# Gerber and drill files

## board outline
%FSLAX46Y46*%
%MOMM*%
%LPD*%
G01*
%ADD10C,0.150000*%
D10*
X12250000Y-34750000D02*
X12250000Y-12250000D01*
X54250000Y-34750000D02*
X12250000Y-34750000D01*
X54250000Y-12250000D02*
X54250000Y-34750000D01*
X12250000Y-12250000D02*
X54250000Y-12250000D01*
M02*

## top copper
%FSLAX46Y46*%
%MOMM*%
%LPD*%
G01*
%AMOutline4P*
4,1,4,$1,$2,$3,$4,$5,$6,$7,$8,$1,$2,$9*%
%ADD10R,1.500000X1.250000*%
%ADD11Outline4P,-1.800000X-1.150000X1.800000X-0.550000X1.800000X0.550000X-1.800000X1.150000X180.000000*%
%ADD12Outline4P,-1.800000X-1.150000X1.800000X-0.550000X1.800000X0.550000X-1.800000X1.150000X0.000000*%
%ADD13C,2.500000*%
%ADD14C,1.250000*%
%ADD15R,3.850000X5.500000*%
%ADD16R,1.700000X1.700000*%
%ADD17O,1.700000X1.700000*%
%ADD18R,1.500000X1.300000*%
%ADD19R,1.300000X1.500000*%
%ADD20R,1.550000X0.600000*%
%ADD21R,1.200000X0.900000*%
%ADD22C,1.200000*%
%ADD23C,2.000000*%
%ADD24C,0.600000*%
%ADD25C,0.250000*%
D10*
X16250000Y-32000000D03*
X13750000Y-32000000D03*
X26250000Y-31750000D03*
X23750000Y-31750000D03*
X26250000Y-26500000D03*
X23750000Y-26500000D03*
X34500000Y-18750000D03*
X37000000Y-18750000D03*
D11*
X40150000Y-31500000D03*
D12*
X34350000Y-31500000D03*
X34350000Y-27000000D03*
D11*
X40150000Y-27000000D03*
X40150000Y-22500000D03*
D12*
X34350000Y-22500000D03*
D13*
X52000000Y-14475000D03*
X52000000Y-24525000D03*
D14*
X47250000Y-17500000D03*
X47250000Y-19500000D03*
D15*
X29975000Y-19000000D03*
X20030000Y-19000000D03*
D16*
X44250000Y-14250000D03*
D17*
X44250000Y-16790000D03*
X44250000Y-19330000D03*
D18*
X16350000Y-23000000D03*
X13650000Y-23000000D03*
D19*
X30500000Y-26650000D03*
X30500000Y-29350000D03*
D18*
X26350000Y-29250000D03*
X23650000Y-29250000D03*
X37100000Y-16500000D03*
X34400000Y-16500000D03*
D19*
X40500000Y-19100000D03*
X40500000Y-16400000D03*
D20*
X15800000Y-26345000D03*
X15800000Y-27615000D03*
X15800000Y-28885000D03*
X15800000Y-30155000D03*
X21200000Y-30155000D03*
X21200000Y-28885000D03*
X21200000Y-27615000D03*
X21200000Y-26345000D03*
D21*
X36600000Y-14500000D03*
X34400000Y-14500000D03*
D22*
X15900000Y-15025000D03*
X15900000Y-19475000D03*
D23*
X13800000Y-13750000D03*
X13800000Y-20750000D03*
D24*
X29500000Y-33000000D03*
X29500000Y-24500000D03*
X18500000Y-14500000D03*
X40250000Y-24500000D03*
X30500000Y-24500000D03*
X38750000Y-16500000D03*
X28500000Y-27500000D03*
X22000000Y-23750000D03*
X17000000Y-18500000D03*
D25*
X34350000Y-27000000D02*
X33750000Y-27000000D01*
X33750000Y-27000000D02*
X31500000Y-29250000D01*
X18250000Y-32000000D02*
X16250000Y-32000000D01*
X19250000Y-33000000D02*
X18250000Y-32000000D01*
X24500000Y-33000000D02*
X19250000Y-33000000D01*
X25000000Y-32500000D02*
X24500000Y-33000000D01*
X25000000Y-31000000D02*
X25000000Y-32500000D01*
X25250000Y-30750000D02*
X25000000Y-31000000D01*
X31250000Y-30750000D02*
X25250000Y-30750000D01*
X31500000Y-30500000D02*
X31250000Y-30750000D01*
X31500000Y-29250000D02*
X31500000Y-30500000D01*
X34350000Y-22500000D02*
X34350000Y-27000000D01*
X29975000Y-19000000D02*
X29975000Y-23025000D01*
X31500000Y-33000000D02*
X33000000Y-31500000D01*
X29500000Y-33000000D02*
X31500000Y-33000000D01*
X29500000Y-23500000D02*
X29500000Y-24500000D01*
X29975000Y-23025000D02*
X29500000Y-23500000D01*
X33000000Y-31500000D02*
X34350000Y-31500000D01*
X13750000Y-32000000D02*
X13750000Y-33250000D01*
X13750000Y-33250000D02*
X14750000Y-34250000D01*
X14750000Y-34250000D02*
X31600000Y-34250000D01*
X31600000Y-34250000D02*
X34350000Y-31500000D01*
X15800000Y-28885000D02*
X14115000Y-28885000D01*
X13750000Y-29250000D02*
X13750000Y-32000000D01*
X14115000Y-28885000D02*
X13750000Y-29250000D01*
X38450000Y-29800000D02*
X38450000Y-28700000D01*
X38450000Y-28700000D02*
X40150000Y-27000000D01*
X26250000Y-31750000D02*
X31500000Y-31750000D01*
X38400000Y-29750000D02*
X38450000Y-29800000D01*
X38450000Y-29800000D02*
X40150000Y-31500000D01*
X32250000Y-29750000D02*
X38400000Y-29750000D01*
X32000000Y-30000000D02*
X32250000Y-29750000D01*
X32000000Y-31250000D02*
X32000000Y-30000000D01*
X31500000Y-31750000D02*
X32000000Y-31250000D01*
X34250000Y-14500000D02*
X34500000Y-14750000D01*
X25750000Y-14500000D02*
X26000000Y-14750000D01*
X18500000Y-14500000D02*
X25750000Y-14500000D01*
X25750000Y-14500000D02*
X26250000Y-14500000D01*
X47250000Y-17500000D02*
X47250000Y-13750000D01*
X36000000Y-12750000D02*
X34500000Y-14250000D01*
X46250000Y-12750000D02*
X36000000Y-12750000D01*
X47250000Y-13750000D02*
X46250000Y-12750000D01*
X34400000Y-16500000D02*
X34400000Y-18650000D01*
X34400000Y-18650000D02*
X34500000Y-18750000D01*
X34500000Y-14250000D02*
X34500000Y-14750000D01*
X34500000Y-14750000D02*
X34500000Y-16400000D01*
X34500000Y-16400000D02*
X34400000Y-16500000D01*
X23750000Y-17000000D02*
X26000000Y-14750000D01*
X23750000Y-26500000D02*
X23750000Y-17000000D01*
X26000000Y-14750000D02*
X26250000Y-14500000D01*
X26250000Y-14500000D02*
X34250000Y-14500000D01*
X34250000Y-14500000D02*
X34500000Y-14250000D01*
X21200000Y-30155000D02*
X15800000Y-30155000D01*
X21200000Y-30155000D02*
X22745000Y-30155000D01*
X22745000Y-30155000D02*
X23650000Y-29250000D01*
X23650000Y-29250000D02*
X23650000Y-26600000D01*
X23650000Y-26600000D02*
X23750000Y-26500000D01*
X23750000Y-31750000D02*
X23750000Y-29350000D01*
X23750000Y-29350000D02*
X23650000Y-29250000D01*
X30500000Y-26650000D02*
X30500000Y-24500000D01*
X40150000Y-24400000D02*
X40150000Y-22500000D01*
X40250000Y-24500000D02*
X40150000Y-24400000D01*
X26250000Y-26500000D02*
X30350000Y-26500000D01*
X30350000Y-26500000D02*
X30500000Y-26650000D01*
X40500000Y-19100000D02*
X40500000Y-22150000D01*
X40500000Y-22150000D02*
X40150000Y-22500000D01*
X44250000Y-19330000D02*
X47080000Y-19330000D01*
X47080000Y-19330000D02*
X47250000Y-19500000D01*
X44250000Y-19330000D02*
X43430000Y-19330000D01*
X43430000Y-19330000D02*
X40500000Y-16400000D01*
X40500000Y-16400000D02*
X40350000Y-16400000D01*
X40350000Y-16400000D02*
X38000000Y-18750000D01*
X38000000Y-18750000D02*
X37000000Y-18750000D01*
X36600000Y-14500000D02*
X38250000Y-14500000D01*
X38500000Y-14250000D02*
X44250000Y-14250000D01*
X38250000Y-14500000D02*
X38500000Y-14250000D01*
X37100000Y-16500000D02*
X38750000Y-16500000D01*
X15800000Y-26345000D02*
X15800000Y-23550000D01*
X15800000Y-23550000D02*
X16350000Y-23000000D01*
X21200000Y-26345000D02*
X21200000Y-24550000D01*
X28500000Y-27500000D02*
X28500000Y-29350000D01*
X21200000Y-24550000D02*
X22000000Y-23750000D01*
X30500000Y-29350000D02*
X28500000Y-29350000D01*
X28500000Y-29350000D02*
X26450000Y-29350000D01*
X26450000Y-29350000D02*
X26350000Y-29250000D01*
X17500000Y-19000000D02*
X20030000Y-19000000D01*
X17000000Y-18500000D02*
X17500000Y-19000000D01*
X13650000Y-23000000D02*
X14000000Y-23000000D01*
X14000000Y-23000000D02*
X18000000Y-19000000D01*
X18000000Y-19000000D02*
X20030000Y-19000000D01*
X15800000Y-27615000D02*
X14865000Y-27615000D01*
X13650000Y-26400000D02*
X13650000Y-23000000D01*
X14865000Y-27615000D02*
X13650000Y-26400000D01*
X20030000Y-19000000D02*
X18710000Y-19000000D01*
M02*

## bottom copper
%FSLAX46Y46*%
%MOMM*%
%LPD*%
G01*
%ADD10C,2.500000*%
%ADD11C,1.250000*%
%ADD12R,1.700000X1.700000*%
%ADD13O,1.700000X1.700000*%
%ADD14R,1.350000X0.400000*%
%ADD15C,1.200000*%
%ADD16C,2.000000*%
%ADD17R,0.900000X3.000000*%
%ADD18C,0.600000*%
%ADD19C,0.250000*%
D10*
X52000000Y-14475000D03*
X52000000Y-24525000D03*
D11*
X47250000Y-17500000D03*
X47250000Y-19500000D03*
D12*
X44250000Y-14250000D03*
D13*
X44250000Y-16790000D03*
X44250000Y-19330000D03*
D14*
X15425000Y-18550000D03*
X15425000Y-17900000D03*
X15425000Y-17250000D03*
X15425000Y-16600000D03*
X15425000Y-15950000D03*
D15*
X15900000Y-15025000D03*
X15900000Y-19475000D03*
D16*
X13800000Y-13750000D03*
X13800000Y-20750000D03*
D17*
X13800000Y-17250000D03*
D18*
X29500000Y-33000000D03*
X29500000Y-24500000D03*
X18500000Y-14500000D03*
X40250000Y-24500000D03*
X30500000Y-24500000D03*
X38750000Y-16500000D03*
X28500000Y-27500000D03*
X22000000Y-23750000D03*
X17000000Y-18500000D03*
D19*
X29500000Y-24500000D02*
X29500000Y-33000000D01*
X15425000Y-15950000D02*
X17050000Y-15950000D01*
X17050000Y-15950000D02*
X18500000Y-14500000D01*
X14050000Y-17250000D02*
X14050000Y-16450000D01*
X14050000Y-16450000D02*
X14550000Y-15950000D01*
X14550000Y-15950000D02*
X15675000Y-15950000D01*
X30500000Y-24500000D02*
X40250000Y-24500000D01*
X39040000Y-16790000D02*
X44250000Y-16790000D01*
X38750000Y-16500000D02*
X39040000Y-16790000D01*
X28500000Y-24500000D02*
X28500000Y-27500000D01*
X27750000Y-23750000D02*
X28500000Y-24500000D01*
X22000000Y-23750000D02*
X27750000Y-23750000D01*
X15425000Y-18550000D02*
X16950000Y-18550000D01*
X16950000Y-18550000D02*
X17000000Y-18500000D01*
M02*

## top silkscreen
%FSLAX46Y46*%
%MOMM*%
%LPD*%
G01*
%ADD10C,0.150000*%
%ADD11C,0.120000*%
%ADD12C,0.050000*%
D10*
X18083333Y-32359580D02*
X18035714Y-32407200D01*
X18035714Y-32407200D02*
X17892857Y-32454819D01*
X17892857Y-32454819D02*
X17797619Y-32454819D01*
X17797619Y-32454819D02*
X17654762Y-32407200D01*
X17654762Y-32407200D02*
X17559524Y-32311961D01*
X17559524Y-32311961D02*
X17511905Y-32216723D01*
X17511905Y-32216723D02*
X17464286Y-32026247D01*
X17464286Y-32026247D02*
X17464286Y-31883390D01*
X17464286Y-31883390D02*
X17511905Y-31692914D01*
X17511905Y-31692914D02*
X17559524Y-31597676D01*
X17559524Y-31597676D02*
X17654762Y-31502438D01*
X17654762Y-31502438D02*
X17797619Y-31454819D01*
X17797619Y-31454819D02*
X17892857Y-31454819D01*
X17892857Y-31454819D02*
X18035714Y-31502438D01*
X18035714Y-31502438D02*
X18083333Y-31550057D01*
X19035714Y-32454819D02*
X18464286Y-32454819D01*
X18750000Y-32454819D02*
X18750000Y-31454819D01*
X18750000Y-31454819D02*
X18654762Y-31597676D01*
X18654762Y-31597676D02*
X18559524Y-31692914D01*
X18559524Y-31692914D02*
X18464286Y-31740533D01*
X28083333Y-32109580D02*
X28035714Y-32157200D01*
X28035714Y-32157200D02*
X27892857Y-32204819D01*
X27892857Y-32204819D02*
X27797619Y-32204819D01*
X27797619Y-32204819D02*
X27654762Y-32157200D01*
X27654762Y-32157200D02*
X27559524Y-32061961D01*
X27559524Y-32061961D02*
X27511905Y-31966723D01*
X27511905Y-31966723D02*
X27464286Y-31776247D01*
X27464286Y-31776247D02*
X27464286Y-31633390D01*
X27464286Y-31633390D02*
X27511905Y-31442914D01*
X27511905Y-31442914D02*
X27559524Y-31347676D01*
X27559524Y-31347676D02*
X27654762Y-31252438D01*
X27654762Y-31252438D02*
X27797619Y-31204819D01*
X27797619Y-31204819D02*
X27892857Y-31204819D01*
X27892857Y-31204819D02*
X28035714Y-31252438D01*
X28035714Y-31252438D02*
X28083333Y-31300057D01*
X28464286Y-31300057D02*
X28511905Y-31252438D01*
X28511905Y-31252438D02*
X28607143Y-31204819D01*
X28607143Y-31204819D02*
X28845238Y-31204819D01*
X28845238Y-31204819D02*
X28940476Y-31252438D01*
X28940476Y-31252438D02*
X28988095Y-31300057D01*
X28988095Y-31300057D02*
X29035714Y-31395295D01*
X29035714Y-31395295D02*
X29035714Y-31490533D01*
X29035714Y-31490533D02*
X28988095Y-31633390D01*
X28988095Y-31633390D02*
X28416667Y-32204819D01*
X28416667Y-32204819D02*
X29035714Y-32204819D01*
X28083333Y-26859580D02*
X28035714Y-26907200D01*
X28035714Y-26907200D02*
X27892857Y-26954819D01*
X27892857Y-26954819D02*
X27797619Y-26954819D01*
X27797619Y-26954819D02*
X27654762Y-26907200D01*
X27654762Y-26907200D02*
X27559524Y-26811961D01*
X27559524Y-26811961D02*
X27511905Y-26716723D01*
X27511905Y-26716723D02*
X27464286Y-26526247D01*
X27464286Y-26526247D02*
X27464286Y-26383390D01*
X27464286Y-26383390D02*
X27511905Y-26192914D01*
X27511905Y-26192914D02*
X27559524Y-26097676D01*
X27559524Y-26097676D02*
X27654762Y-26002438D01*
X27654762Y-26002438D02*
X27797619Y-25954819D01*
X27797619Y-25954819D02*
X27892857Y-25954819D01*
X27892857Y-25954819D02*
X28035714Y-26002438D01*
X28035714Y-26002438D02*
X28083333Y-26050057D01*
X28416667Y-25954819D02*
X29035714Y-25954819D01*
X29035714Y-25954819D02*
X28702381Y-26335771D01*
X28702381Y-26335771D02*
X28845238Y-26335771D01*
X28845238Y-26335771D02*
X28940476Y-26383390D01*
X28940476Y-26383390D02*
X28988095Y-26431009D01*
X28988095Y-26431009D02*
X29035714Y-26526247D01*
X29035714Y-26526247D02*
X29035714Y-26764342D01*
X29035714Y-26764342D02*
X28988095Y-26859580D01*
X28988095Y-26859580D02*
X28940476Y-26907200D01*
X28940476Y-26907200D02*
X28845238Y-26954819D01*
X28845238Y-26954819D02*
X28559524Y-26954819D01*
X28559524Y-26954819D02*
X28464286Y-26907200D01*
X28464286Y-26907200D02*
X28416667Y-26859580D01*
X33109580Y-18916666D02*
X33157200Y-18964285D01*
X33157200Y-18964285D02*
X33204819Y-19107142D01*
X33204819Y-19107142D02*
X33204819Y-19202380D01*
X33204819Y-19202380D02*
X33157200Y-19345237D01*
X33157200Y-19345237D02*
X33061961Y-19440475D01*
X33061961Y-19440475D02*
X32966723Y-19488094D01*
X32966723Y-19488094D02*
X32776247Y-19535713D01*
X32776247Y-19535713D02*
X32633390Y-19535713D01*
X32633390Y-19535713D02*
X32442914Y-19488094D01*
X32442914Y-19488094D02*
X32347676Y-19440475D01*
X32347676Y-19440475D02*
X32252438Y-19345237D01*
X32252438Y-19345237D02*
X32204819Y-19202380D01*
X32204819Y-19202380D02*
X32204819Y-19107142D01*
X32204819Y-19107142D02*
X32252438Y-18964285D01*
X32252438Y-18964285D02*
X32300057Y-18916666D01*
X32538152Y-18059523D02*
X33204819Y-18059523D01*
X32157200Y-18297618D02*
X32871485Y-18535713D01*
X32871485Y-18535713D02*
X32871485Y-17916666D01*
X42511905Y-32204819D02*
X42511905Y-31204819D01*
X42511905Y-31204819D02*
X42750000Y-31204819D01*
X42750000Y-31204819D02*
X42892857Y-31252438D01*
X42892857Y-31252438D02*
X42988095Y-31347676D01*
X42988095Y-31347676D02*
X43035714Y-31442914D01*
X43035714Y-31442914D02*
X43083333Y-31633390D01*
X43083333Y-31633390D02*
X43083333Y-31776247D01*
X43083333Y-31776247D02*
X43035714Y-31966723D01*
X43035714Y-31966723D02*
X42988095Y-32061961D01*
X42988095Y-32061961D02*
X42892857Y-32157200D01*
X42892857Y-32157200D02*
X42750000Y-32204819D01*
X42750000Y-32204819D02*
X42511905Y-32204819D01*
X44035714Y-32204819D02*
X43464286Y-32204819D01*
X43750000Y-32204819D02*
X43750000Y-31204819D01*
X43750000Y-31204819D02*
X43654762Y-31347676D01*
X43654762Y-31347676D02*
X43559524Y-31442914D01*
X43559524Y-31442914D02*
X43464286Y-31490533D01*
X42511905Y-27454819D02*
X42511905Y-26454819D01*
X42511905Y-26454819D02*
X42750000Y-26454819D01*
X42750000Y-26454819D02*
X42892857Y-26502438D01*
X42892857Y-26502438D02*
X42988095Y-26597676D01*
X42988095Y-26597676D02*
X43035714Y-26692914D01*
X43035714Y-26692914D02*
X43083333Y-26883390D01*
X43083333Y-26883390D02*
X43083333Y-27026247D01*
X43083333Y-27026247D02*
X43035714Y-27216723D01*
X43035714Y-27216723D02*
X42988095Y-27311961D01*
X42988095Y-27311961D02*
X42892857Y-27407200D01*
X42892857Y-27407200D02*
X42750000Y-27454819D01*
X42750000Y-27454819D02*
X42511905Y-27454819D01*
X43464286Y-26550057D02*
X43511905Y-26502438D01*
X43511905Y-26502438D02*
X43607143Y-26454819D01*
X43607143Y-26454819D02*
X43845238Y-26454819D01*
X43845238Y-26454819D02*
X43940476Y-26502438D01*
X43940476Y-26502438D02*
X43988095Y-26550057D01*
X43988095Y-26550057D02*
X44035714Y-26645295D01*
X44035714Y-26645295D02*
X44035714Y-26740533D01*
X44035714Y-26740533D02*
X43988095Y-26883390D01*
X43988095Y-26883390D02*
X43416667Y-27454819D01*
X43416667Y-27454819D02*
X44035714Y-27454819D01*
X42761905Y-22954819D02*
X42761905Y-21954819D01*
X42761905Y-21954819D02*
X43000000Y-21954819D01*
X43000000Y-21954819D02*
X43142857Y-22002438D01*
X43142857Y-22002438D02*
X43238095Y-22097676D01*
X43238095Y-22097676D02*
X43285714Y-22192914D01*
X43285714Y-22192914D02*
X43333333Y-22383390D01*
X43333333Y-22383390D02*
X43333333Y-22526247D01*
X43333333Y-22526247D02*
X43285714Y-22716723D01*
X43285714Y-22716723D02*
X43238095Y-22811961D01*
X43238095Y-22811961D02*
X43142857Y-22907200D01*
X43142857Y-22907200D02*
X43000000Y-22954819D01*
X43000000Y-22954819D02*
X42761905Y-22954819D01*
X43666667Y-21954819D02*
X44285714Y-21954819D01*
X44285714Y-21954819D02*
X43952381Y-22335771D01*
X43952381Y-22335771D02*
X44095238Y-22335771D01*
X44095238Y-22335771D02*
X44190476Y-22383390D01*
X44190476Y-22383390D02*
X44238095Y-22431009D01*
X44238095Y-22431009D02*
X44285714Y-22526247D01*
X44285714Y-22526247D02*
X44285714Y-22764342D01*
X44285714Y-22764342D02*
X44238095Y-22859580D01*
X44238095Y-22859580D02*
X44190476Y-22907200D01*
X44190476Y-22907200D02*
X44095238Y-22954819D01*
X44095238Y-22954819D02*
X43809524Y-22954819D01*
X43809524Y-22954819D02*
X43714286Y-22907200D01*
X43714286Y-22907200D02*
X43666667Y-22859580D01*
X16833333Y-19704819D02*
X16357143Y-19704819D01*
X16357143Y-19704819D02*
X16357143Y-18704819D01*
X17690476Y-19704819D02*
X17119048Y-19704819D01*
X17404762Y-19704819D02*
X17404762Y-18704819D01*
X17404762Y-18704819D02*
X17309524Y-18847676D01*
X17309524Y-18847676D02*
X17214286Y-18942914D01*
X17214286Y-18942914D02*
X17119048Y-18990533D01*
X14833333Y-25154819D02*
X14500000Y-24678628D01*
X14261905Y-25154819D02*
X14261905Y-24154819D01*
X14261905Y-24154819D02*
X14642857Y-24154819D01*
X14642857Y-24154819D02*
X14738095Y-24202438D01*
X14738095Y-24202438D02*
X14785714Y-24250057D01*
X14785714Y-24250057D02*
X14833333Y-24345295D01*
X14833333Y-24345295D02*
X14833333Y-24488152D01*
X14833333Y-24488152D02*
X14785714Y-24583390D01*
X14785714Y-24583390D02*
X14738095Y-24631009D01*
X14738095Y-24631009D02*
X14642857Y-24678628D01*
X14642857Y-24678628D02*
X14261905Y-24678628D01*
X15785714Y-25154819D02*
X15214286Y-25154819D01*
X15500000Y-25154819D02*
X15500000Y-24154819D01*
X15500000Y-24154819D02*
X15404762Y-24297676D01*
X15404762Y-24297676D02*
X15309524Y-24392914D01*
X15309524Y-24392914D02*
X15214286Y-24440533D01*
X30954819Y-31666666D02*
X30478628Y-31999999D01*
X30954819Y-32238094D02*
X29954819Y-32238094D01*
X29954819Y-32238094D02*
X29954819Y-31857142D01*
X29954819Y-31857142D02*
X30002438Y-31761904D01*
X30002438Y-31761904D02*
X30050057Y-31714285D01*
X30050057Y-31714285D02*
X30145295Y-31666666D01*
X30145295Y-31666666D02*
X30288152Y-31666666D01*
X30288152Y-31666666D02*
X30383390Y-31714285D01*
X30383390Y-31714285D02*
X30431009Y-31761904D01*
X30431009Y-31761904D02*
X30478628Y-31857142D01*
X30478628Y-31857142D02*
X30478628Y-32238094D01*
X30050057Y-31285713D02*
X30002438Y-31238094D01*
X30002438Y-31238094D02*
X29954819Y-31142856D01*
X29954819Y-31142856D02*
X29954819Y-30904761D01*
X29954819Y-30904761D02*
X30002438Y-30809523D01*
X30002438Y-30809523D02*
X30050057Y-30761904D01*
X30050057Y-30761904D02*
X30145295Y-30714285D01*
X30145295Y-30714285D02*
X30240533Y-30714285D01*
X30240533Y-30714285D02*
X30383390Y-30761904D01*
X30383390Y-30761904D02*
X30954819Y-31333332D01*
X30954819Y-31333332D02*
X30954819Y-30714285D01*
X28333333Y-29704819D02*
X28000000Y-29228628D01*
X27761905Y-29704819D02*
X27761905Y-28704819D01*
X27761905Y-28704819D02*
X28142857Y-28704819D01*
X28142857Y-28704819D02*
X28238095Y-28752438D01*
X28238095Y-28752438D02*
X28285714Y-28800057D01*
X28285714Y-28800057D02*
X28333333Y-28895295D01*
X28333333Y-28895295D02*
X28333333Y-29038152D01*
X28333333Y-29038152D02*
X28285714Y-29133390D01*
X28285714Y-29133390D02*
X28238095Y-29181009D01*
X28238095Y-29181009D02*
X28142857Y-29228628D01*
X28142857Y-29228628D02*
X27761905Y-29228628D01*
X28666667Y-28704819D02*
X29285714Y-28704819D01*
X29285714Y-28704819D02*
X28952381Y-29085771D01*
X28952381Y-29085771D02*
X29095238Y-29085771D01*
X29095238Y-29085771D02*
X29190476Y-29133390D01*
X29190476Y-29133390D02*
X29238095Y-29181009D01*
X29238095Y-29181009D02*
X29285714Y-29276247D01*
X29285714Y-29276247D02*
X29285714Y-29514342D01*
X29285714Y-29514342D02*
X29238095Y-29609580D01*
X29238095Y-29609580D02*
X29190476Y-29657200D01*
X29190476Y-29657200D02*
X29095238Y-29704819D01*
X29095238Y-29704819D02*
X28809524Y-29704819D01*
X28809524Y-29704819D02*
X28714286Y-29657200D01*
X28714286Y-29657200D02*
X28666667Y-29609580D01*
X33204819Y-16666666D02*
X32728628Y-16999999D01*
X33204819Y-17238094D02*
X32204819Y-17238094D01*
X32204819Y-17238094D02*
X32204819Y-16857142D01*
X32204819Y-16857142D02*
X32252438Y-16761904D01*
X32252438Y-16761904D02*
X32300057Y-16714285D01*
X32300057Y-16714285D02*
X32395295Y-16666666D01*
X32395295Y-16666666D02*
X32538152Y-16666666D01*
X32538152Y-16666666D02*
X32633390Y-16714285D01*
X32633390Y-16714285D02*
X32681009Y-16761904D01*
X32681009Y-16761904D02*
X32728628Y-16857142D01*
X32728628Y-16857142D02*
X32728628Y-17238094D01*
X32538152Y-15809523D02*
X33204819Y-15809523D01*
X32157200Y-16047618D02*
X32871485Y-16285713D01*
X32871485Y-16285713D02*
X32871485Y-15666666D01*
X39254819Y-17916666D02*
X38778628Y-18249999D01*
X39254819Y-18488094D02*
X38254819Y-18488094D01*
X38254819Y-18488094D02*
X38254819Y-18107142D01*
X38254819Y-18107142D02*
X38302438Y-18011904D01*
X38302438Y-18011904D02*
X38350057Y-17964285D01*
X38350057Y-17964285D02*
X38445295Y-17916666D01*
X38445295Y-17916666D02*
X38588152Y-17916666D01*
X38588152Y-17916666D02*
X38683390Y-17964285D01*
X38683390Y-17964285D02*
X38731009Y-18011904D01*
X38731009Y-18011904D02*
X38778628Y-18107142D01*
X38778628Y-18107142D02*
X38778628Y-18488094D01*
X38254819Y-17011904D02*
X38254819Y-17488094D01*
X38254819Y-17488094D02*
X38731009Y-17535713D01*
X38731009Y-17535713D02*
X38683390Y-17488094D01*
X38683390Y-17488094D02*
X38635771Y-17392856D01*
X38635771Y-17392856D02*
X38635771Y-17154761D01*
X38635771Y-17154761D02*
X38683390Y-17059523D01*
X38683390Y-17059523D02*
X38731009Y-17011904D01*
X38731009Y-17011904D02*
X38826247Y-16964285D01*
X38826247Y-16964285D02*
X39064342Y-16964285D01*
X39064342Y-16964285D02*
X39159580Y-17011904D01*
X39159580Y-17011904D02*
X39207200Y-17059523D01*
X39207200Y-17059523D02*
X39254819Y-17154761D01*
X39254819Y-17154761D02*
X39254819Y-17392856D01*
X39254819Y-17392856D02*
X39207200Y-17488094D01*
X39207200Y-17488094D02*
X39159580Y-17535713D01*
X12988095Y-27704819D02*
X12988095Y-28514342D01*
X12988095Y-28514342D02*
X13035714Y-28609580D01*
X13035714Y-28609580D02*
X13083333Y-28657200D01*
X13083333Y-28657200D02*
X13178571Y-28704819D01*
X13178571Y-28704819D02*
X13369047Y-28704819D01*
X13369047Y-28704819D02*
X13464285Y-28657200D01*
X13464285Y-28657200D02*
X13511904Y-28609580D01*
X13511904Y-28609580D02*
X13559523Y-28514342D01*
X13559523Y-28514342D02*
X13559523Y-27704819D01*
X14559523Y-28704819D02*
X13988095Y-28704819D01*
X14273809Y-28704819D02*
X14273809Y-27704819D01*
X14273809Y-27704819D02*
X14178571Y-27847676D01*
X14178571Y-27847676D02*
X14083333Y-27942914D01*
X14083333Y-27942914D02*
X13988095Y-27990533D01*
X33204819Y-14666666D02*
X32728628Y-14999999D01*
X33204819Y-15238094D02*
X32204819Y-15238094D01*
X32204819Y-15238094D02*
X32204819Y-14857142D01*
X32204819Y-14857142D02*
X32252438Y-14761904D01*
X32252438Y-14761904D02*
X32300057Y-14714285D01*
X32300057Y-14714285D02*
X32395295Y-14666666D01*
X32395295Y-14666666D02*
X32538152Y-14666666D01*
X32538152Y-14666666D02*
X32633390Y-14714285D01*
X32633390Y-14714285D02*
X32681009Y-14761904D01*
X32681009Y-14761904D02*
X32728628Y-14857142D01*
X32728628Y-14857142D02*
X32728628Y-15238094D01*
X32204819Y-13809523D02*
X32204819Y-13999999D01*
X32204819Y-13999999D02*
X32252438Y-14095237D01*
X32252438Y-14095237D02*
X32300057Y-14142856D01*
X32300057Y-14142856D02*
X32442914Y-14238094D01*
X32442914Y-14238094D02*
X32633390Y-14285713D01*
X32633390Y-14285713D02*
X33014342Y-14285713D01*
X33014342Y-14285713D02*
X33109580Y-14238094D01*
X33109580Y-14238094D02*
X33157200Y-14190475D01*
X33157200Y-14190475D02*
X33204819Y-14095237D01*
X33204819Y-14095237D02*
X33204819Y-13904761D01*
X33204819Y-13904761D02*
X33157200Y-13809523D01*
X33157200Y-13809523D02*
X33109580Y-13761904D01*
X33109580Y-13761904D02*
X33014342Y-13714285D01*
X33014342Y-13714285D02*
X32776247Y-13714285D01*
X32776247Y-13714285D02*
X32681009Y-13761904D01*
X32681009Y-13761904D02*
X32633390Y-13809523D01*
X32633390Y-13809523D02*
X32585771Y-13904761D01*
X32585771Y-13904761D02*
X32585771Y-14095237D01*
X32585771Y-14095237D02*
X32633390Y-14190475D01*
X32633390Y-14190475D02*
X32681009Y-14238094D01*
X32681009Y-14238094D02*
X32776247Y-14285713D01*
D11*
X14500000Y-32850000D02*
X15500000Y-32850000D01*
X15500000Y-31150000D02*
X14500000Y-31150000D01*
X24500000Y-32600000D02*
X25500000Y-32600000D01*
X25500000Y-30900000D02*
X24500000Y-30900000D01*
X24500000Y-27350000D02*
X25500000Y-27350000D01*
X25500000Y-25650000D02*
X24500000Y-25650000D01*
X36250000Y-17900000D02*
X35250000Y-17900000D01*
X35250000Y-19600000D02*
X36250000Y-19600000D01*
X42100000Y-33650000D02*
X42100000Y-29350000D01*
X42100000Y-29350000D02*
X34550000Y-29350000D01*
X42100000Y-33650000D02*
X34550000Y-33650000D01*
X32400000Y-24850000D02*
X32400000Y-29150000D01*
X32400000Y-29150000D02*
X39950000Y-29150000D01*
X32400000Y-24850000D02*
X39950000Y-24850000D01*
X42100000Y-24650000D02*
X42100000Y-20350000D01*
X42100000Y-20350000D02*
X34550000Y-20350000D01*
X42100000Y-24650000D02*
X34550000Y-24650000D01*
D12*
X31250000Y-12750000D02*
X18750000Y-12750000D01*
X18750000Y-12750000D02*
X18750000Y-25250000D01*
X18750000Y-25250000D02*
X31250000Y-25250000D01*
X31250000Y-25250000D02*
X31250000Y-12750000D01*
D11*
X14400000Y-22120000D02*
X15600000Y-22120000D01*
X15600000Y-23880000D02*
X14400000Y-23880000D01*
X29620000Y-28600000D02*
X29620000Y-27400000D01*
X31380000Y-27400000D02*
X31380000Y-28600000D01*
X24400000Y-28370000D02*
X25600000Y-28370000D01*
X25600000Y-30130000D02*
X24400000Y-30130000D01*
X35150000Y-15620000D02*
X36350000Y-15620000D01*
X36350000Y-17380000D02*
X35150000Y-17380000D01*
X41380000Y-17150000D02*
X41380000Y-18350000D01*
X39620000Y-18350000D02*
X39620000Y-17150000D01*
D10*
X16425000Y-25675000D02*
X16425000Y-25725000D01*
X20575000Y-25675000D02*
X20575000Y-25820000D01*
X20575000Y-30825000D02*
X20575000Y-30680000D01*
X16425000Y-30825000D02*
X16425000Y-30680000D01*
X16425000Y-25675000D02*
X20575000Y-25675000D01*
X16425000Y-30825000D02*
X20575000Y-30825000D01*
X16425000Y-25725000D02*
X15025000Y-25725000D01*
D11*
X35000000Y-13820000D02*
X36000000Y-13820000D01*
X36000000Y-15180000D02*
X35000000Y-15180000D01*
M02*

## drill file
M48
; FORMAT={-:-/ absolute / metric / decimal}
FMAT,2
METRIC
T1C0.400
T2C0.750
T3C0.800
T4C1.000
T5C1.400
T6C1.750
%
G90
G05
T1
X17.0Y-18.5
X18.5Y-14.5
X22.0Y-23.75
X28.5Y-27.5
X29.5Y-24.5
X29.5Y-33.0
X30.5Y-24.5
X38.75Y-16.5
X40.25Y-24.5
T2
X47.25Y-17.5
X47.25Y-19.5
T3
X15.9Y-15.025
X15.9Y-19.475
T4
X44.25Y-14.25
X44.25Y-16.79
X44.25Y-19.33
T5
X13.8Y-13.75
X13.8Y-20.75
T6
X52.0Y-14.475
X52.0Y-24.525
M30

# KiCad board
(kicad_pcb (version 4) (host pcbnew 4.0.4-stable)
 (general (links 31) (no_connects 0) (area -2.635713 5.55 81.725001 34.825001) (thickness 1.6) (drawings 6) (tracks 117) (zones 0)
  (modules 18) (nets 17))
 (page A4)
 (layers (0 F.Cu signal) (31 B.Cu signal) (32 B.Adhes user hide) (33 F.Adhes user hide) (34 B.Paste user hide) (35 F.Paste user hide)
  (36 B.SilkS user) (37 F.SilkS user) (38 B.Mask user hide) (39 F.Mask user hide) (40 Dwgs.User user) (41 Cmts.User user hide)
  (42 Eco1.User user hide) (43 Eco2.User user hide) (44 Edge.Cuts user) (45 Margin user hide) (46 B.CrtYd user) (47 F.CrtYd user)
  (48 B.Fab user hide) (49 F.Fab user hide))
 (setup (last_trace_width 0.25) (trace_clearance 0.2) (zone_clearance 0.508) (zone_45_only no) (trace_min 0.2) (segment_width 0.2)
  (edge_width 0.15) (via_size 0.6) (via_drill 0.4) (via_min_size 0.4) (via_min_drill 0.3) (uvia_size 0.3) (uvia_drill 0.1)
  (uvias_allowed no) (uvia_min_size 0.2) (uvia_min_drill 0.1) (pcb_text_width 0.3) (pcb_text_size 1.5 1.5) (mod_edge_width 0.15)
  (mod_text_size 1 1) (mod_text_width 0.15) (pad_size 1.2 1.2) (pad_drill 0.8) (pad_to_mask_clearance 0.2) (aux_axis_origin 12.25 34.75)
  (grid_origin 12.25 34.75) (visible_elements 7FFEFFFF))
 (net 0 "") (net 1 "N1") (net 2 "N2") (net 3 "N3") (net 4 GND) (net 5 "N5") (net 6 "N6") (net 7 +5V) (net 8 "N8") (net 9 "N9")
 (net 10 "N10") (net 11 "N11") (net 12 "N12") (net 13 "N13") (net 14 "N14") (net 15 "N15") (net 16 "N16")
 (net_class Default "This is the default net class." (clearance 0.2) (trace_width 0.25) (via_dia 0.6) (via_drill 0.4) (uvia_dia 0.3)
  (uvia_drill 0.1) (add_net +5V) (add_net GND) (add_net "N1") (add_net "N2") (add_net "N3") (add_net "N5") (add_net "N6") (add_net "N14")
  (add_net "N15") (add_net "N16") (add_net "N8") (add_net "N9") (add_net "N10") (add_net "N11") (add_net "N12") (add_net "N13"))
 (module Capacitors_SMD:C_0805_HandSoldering (layer F.Cu) (at 15 32 180)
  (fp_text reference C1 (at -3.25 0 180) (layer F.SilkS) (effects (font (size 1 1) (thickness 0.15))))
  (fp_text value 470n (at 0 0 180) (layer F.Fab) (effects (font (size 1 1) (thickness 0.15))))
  (fp_line (start 0.5 -0.85) (end -0.5 -0.85) (layer F.SilkS) (width 0.12))
  (fp_line (start -0.5 0.85) (end 0.5 0.85) (layer F.SilkS) (width 0.12))
  (pad 1 smd rect (at -1.25 0 180) (size 1.5 1.25) (layers F.Cu F.Paste F.Mask) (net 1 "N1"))
  (pad 2 smd rect (at 1.25 0 180) (size 1.5 1.25) (layers F.Cu F.Paste F.Mask) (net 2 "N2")))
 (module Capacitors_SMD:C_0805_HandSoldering (layer F.Cu) (at 25 31.75 180)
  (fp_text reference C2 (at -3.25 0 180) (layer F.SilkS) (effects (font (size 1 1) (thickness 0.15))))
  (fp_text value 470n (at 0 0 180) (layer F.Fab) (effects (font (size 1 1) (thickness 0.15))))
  (fp_line (start 0.5 -0.85) (end -0.5 -0.85) (layer F.SilkS) (width 0.12))
  (fp_line (start -0.5 0.85) (end 0.5 0.85) (layer F.SilkS) (width 0.12))
  (pad 1 smd rect (at -1.25 0 180) (size 1.5 1.25) (layers F.Cu F.Paste F.Mask) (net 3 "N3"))
  (pad 2 smd rect (at 1.25 0 180) (size 1.5 1.25) (layers F.Cu F.Paste F.Mask) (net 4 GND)))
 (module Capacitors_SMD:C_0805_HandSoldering (layer F.Cu) (at 25 26.5 180)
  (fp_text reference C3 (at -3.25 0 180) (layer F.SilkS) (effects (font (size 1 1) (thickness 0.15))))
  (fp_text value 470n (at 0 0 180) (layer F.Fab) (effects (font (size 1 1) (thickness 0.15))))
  (fp_line (start 0.5 -0.85) (end -0.5 -0.85) (layer F.SilkS) (width 0.12))
  (fp_line (start -0.5 0.85) (end 0.5 0.85) (layer F.SilkS) (width 0.12))
  (pad 1 smd rect (at -1.25 0 180) (size 1.5 1.25) (layers F.Cu F.Paste F.Mask) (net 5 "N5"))
  (pad 2 smd rect (at 1.25 0 180) (size 1.5 1.25) (layers F.Cu F.Paste F.Mask) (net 4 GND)))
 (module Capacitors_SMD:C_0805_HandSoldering (layer F.Cu) (at 35.75 18.75)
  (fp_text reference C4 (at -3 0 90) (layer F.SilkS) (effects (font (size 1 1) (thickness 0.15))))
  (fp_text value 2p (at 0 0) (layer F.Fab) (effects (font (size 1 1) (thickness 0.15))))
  (fp_line (start 0.5 -0.85) (end -0.5 -0.85) (layer F.SilkS) (width 0.12))
  (fp_line (start -0.5 0.85) (end 0.5 0.85) (layer F.SilkS) (width 0.12))
  (pad 1 smd rect (at -1.25 0) (size 1.5 1.25) (layers F.Cu F.Paste F.Mask) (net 4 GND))
  (pad 2 smd rect (at 1.25 0) (size 1.5 1.25) (layers F.Cu F.Paste F.Mask) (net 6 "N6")))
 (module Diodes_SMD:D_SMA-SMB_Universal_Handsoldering (layer F.Cu) (at 37.25 31.5 180)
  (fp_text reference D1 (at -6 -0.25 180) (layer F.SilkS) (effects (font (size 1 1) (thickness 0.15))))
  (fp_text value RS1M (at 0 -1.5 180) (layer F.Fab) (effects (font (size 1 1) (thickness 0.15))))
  (fp_line (start -4.85 -2.15) (end -4.85 2.15) (layer F.SilkS) (width 0.12))
  (fp_line (start -4.85 2.15) (end 2.7 2.15) (layer F.SilkS) (width 0.12))
  (fp_line (start -4.85 -2.15) (end 2.7 -2.15) (layer F.SilkS) (width 0.12))
  (pad 1 smd trapezoid (at -2.9 0 180) (size 3.6 1.7) (rect_delta 0.6 0) (layers F.Cu F.Paste F.Mask) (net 3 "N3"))
  (pad 2 smd trapezoid (at 2.9 0) (size 3.6 1.7) (rect_delta 0.6 0) (layers F.Cu F.Paste F.Mask) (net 2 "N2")))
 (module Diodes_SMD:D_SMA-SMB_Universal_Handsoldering (layer F.Cu) (at 37.25 27)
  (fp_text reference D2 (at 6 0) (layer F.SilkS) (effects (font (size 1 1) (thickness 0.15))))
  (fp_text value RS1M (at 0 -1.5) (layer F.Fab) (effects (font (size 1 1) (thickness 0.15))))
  (fp_line (start -4.85 -2.15) (end -4.85 2.15) (layer F.SilkS) (width 0.12))
  (fp_line (start -4.85 2.15) (end 2.7 2.15) (layer F.SilkS) (width 0.12))
  (fp_line (start -4.85 -2.15) (end 2.7 -2.15) (layer F.SilkS) (width 0.12))
  (pad 1 smd trapezoid (at -2.9 0) (size 3.6 1.7) (rect_delta 0.6 0) (layers F.Cu F.Paste F.Mask) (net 1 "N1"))
  (pad 2 smd trapezoid (at 2.9 0 180) (size 3.6 1.7) (rect_delta 0.6 0) (layers F.Cu F.Paste F.Mask) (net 3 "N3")))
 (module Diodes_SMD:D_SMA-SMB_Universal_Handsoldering (layer F.Cu) (at 37.25 22.5 180)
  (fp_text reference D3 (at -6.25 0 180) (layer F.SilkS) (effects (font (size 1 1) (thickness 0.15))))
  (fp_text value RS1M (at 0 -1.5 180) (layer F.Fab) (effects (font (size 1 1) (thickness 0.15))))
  (fp_line (start -4.85 -2.15) (end -4.85 2.15) (layer F.SilkS) (width 0.12))
  (fp_line (start -4.85 2.15) (end 2.7 2.15) (layer F.SilkS) (width 0.12))
  (fp_line (start -4.85 -2.15) (end 2.7 -2.15) (layer F.SilkS) (width 0.12))
  (pad 1 smd trapezoid (at -2.9 0 180) (size 3.6 1.7) (rect_delta 0.6 0) (layers F.Cu F.Paste F.Mask) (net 5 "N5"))
  (pad 2 smd trapezoid (at 2.9 0) (size 3.6 1.7) (rect_delta 0.6 0) (layers F.Cu F.Paste F.Mask) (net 1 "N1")))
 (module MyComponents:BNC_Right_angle (layer B.Cu) (at 52 19.5 270)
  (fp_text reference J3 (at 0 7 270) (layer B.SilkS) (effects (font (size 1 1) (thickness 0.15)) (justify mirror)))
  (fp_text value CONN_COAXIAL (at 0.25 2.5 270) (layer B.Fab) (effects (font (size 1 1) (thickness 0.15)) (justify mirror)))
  (pad 3 thru_hole circle (at -5.025 0 270) (size 2.5 2.5) (drill 1.75) (layers *.Cu *.Mask))
  (pad 3 thru_hole circle (at 5.025 0 270) (size 2.5 2.5) (drill 1.75) (layers *.Cu *.Mask))
  (pad 2 thru_hole circle (at -2 4.75 270) (size 1.25 1.25) (drill 0.75) (layers *.Cu *.Mask) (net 4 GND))
  (pad 1 thru_hole circle (at 0 4.75 270) (size 1.25 1.25) (drill 0.75) (layers *.Cu *.Mask) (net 6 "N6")))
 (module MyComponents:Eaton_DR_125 (layer F.Cu) (at 25 19 180)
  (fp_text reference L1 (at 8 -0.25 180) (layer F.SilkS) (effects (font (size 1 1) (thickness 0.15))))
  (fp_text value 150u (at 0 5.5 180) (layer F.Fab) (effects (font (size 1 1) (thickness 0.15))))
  (fp_line (start -6.25 6.25) (end 6.25 6.25) (layer F.SilkS) (width 0.05))
  (fp_line (start 6.25 6.25) (end 6.25 -6.25) (layer F.SilkS) (width 0.05))
  (fp_line (start 6.25 -6.25) (end -6.25 -6.25) (layer F.SilkS) (width 0.05))
  (fp_line (start -6.25 -6.25) (end -6.25 6.25) (layer F.SilkS) (width 0.05))
  (pad 1 smd rect (at -4.975 0 180) (size 3.85 5.5) (layers F.Cu F.Paste F.Mask) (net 2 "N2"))
  (pad 2 smd rect (at 4.97 0 180) (size 3.85 5.5) (layers F.Cu F.Paste F.Mask) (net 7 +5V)))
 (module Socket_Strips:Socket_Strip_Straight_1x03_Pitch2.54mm (layer B.Cu) (at 44.25 14.25 180)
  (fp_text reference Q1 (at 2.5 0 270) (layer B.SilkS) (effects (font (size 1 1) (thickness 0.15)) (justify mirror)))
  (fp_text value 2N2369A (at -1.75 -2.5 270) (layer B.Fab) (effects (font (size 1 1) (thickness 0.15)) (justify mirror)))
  (pad 1 thru_hole rect (at 0 0 180) (size 1.7 1.7) (drill 1) (layers *.Cu *.Mask) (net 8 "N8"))
  (pad 2 thru_hole oval (at 0 -2.54 180) (size 1.7 1.7) (drill 1) (layers *.Cu *.Mask) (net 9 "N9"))
  (pad 3 thru_hole oval (at 0 -5.08 180) (size 1.7 1.7) (drill 1) (layers *.Cu *.Mask) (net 6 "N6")))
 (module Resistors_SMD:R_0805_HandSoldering (layer F.Cu) (at 15 23 180)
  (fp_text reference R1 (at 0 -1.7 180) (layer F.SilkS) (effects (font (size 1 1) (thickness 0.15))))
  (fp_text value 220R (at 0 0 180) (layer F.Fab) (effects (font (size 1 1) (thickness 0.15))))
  (fp_line (start 0.6 0.88) (end -0.6 0.88) (layer F.SilkS) (width 0.12))
  (fp_line (start -0.6 -0.88) (end 0.6 -0.88) (layer F.SilkS) (width 0.12))
  (pad 1 smd rect (at -1.35 0 180) (size 1.5 1.3) (layers F.Cu F.Paste F.Mask) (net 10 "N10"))
  (pad 2 smd rect (at 1.35 0 180) (size 1.5 1.3) (layers F.Cu F.Paste F.Mask) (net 7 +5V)))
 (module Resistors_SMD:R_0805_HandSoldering (layer F.Cu) (at 30.5 28 270)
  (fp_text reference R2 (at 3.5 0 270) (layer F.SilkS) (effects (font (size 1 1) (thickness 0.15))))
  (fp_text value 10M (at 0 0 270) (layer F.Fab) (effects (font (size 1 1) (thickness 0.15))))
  (fp_line (start 0.6 0.88) (end -0.6 0.88) (layer F.SilkS) (width 0.12))
  (fp_line (start -0.6 -0.88) (end 0.6 -0.88) (layer F.SilkS) (width 0.12))
  (pad 1 smd rect (at -1.35 0 270) (size 1.5 1.3) (layers F.Cu F.Paste F.Mask) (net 5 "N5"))
  (pad 2 smd rect (at 1.35 0 270) (size 1.5 1.3) (layers F.Cu F.Paste F.Mask) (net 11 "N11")))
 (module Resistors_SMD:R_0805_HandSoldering (layer F.Cu) (at 25 29.25 180)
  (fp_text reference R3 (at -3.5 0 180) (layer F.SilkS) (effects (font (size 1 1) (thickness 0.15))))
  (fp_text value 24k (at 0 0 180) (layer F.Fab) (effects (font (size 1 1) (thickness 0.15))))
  (fp_line (start 0.6 0.88) (end -0.6 0.88) (layer F.SilkS) (width 0.12))
  (fp_line (start -0.6 -0.88) (end 0.6 -0.88) (layer F.SilkS) (width 0.12))
  (pad 1 smd rect (at -1.35 0 180) (size 1.5 1.3) (layers F.Cu F.Paste F.Mask) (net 11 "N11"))
  (pad 2 smd rect (at 1.35 0 180) (size 1.5 1.3) (layers F.Cu F.Paste F.Mask) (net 4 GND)))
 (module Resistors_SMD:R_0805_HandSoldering (layer F.Cu) (at 35.75 16.5 180)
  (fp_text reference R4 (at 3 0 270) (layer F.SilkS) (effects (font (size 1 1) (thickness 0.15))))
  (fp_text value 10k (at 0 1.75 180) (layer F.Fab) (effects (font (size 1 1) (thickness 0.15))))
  (fp_line (start 0.6 0.88) (end -0.6 0.88) (layer F.SilkS) (width 0.12))
  (fp_line (start -0.6 -0.88) (end 0.6 -0.88) (layer F.SilkS) (width 0.12))
  (pad 1 smd rect (at -1.35 0 180) (size 1.5 1.3) (layers F.Cu F.Paste F.Mask) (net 9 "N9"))
  (pad 2 smd rect (at 1.35 0 180) (size 1.5 1.3) (layers F.Cu F.Paste F.Mask) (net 4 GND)))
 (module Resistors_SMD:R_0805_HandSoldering (layer F.Cu) (at 40.5 17.75 90)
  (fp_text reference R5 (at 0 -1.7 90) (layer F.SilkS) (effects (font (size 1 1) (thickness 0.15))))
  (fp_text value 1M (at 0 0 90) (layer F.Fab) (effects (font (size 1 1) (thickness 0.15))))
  (fp_line (start 0.6 0.88) (end -0.6 0.88) (layer F.SilkS) (width 0.12))
  (fp_line (start -0.6 -0.88) (end 0.6 -0.88) (layer F.SilkS) (width 0.12))
  (pad 1 smd rect (at -1.35 0 90) (size 1.5 1.3) (layers F.Cu F.Paste F.Mask) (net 5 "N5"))
  (pad 2 smd rect (at 1.35 0 90) (size 1.5 1.3) (layers F.Cu F.Paste F.Mask) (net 6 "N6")))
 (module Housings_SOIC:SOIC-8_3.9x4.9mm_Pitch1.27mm (layer F.Cu) (at 18.5 28.25)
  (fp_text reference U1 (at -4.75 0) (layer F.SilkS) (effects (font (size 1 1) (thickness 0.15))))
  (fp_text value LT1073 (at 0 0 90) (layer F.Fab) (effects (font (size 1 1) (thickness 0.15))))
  (fp_line (start -2.075 -2.575) (end -2.075 -2.525) (layer F.SilkS) (width 0.15))
  (fp_line (start 2.075 -2.575) (end 2.075 -2.43) (layer F.SilkS) (width 0.15))
  (fp_line (start 2.075 2.575) (end 2.075 2.43) (layer F.SilkS) (width 0.15))
  (fp_line (start -2.075 2.575) (end -2.075 2.43) (layer F.SilkS) (width 0.15))
  (fp_line (start -2.075 -2.575) (end 2.075 -2.575) (layer F.SilkS) (width 0.15))
  (fp_line (start -2.075 2.575) (end 2.075 2.575) (layer F.SilkS) (width 0.15))
  (fp_line (start -2.075 -2.525) (end -3.475 -2.525) (layer F.SilkS) (width 0.15))
  (pad 1 smd rect (at -2.7 -1.905) (size 1.55 0.6) (layers F.Cu F.Paste F.Mask) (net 10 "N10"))
  (pad 2 smd rect (at -2.7 -0.635) (size 1.55 0.6) (layers F.Cu F.Paste F.Mask) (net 7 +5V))
  (pad 3 smd rect (at -2.7 0.635) (size 1.55 0.6) (layers F.Cu F.Paste F.Mask) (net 2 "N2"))
  (pad 4 smd rect (at -2.7 1.905) (size 1.55 0.6) (layers F.Cu F.Paste F.Mask) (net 4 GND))
  (pad 5 smd rect (at 2.7 1.905) (size 1.55 0.6) (layers F.Cu F.Paste F.Mask) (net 4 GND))
  (pad 6 smd rect (at 2.7 0.635) (size 1.55 0.6) (layers F.Cu F.Paste F.Mask) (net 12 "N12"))
  (pad 7 smd rect (at 2.7 -0.635) (size 1.55 0.6) (layers F.Cu F.Paste F.Mask) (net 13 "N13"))
  (pad 8 smd rect (at 2.7 -1.905) (size 1.55 0.6) (layers F.Cu F.Paste F.Mask) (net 11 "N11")))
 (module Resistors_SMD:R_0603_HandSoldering (layer F.Cu) (at 35.5 14.5 180)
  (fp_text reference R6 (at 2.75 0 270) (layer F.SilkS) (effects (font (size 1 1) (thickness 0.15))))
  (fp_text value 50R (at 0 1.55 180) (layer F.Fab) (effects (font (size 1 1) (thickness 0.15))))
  (fp_line (start 0.5 0.68) (end -0.5 0.68) (layer F.SilkS) (width 0.12))
  (fp_line (start -0.5 -0.68) (end 0.5 -0.68) (layer F.SilkS) (width 0.12))
  (pad 1 smd rect (at -1.1 0 180) (size 1.2 0.9) (layers F.Cu F.Paste F.Mask) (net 8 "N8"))
  (pad 2 smd rect (at 1.1 0 180) (size 1.2 0.9) (layers F.Cu F.Paste F.Mask) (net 4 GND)))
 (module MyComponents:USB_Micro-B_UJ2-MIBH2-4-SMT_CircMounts (layer B.Cu) (at 10.75 17.25)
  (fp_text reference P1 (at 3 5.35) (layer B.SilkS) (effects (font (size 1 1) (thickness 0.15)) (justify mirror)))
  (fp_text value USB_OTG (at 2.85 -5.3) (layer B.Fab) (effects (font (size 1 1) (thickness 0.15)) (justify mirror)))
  (pad 1 smd rect (at 4.675 1.3) (size 1.35 0.4) (layers B.Cu B.Paste B.Mask) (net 7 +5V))
  (pad 2 smd rect (at 4.675 0.65) (size 1.35 0.4) (layers B.Cu B.Paste B.Mask) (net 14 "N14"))
  (pad 3 smd rect (at 4.675 0) (size 1.35 0.4) (layers B.Cu B.Paste B.Mask) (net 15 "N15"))
  (pad 4 smd rect (at 4.675 -0.65) (size 1.35 0.4) (layers B.Cu B.Paste B.Mask) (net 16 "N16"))
  (pad 5 smd rect (at 4.675 -1.3) (size 1.35 0.4) (layers B.Cu B.Paste B.Mask) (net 4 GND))
  (pad 7 thru_hole circle (at 5.15 -2.225) (size 1.2 1.2) (drill 0.8) (layers *.Cu *.Mask) (clearance 0.1))
  (pad 7 thru_hole circle (at 5.15 2.225) (size 1.2 1.2) (drill 0.8) (layers *.Cu *.Mask) (clearance 0.1))
  (pad 7 thru_hole circle (at 3.05 -3.5) (size 2 2) (drill 1.4) (layers *.Cu *.Mask))
  (pad 7 thru_hole circle (at 3.05 3.5) (size 2 2) (drill 1.4) (layers *.Cu *.Mask))
  (pad 6 smd rect (at 3.05 0) (size 0.9 3) (layers B.Cu B.Paste B.Mask) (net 4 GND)))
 (gr_line (start 12.25 34.75) (end 12.25 12.25) (angle 90) (layer Edge.Cuts) (width 0.15))
 (gr_line (start 54.25 34.75) (end 12.25 34.75) (angle 90) (layer Edge.Cuts) (width 0.15))
 (gr_line (start 54.25 12.25) (end 54.25 34.75) (angle 90) (layer Edge.Cuts) (width 0.15))
 (gr_line (start 12.25 12.25) (end 54.25 12.25) (angle 90) (layer Edge.Cuts) (width 0.15))
 (segment (start 34.35 27) (end 33.75 27) (width 0.25) (layer F.Cu) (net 1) (status 30))
 (segment (start 33.75 27) (end 31.5 29.25) (width 0.25) (layer F.Cu) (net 1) (status 10))
 (segment (start 18.25 32) (end 16.25 32) (width 0.25) (layer F.Cu) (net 1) (status 20))
 (segment (start 19.25 33) (end 18.25 32) (width 0.25) (layer F.Cu) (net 1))
 (segment (start 24.5 33) (end 19.25 33) (width 0.25) (layer F.Cu) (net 1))
 (segment (start 25 32.5) (end 24.5 33) (width 0.25) (layer F.Cu) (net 1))
 (segment (start 25 31) (end 25 32.5) (width 0.25) (layer F.Cu) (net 1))
 (segment (start 25.25 30.75) (end 25 31) (width 0.25) (layer F.Cu) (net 1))
 (segment (start 31.25 30.75) (end 25.25 30.75) (width 0.25) (layer F.Cu) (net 1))
 (segment (start 31.5 30.5) (end 31.25 30.75) (width 0.25) (layer F.Cu) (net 1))
 (segment (start 31.5 29.25) (end 31.5 30.5) (width 0.25) (layer F.Cu) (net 1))
 (segment (start 34.35 22.5) (end 34.35 27) (width 0.25) (layer F.Cu) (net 1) (status 30))
 (segment (start 29.975 19) (end 29.975 23.025) (width 0.25) (layer F.Cu) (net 2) (status 10))
 (segment (start 31.5 33) (end 33 31.5) (width 0.25) (layer F.Cu) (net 2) (status 20))
 (segment (start 29.5 33) (end 31.5 33) (width 0.25) (layer F.Cu) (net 2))
 (via (at 29.5 33) (size 0.6) (drill 0.4) (layers F.Cu B.Cu) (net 2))
 (segment (start 29.5 24.5) (end 29.5 33) (width 0.25) (layer B.Cu) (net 2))
 (via (at 29.5 24.5) (size 0.6) (drill 0.4) (layers F.Cu B.Cu) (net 2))
 (segment (start 29.5 23.5) (end 29.5 24.5) (width 0.25) (layer F.Cu) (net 2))
 (segment (start 29.975 23.025) (end 29.5 23.5) (width 0.25) (layer F.Cu) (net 2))
 (segment (start 33 31.5) (end 34.35 31.5) (width 0.25) (layer F.Cu) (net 2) (status 30))
 (segment (start 13.75 32) (end 13.75 33.25) (width 0.25) (layer F.Cu) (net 2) (status 10))
 (segment (start 13.75 33.25) (end 14.75 34.25) (width 0.25) (layer F.Cu) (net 2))
 (segment (start 14.75 34.25) (end 31.6 34.25) (width 0.25) (layer F.Cu) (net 2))
 (segment (start 31.6 34.25) (end 34.35 31.5) (width 0.25) (layer F.Cu) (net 2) (status 20))
 (segment (start 15.8 28.885) (end 14.115 28.885) (width 0.25) (layer F.Cu) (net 2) (status 10))
 (segment (start 13.75 29.25) (end 13.75 32) (width 0.25) (layer F.Cu) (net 2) (status 20))
 (segment (start 14.115 28.885) (end 13.75 29.25) (width 0.25) (layer F.Cu) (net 2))
 (segment (start 38.45 29.8) (end 38.45 28.7) (width 0.25) (layer F.Cu) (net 3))
 (segment (start 38.45 28.7) (end 40.15 27) (width 0.25) (layer F.Cu) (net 3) (status 20))
 (segment (start 26.25 31.75) (end 31.5 31.75) (width 0.25) (layer F.Cu) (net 3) (status 10))
 (segment (start 38.4 29.75) (end 38.45 29.8) (width 0.25) (layer F.Cu) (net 3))
 (segment (start 38.45 29.8) (end 40.15 31.5) (width 0.25) (layer F.Cu) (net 3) (status 20))
 (segment (start 32.25 29.75) (end 38.4 29.75) (width 0.25) (layer F.Cu) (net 3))
 (segment (start 32 30) (end 32.25 29.75) (width 0.25) (layer F.Cu) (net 3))
 (segment (start 32 31.25) (end 32 30) (width 0.25) (layer F.Cu) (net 3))
 (segment (start 31.5 31.75) (end 32 31.25) (width 0.25) (layer F.Cu) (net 3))
 (segment (start 34.25 14.5) (end 34.5 14.75) (width 0.25) (layer F.Cu) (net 4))
 (segment (start 25.75 14.5) (end 26 14.75) (width 0.25) (layer F.Cu) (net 4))
 (segment (start 15.425 15.95) (end 17.05 15.95) (width 0.25) (layer B.Cu) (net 4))
 (segment (start 18.5 14.5) (end 25.75 14.5) (width 0.25) (layer F.Cu) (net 4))
 (segment (start 25.75 14.5) (end 26.25 14.5) (width 0.25) (layer F.Cu) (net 4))
 (via (at 18.5 14.5) (size 0.6) (drill 0.4) (layers F.Cu B.Cu) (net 4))
 (segment (start 17.05 15.95) (end 18.5 14.5) (width 0.25) (layer B.Cu) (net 4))
 (segment (start 47.25 17.5) (end 47.25 13.75) (width 0.25) (layer F.Cu) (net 4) (status 10))
 (segment (start 36 12.75) (end 34.5 14.25) (width 0.25) (layer F.Cu) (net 4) (status 20))
 (segment (start 46.25 12.75) (end 36 12.75) (width 0.25) (layer F.Cu) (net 4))
 (segment (start 47.25 13.75) (end 46.25 12.75) (width 0.25) (layer F.Cu) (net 4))
 (segment (start 34.4 16.5) (end 34.4 18.65) (width 0.25) (layer F.Cu) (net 4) (status 30))
 (segment (start 34.4 18.65) (end 34.5 18.75) (width 0.25) (layer F.Cu) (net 4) (status 30))
 (segment (start 34.5 14.25) (end 34.5 14.75) (width 0.25) (layer F.Cu) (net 4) (status 30))
 (segment (start 34.5 14.75) (end 34.5 16.4) (width 0.25) (layer F.Cu) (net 4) (status 30))
 (segment (start 34.5 16.4) (end 34.4 16.5) (width 0.25) (layer F.Cu) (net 4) (status 30))
 (segment (start 23.75 17) (end 26 14.75) (width 0.25) (layer F.Cu) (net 4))
 (segment (start 23.75 26.5) (end 23.75 17) (width 0.25) (layer F.Cu) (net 4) (status 10))
 (segment (start 26 14.75) (end 26.25 14.5) (width 0.25) (layer F.Cu) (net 4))
 (segment (start 26.25 14.5) (end 34.25 14.5) (width 0.25) (layer F.Cu) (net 4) (status 20))
 (segment (start 34.25 14.5) (end 34.5 14.25) (width 0.25) (layer F.Cu) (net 4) (status 30))
 (segment (start 21.2 30.155) (end 15.8 30.155) (width 0.25) (layer F.Cu) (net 4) (status 30))
 (segment (start 21.2 30.155) (end 22.745 30.155) (width 0.25) (layer F.Cu) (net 4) (status 10))
 (segment (start 22.745 30.155) (end 23.65 29.25) (width 0.25) (layer F.Cu) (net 4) (status 20))
 (segment (start 23.65 29.25) (end 23.65 26.6) (width 0.25) (layer F.Cu) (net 4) (status 30))
 (segment (start 23.65 26.6) (end 23.75 26.5) (width 0.25) (layer F.Cu) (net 4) (status 30))
 (segment (start 23.75 31.75) (end 23.75 29.35) (width 0.25) (layer F.Cu) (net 4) (status 30))
 (segment (start 23.75 29.35) (end 23.65 29.25) (width 0.25) (layer F.Cu) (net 4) (status 30))
 (segment (start 14.05 17.25) (end 14.05 16.45) (width 0.25) (layer B.Cu) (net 4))
 (segment (start 14.05 16.45) (end 14.55 15.95) (width 0.25) (layer B.Cu) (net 4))
 (segment (start 14.55 15.95) (end 15.675 15.95) (width 0.25) (layer B.Cu) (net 4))
 (segment (start 30.5 26.65) (end 30.5 24.5) (width 0.25) (layer F.Cu) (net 5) (status 10))
 (segment (start 40.15 24.4) (end 40.15 22.5) (width 0.25) (layer F.Cu) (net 5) (status 20))
 (segment (start 40.25 24.5) (end 40.15 24.4) (width 0.25) (layer F.Cu) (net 5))
 (via (at 40.25 24.5) (size 0.6) (drill 0.4) (layers F.Cu B.Cu) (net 5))
 (segment (start 30.5 24.5) (end 40.25 24.5) (width 0.25) (layer B.Cu) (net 5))
 (via (at 30.5 24.5) (size 0.6) (drill 0.4) (layers F.Cu B.Cu) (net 5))
 (segment (start 26.25 26.5) (end 30.35 26.5) (width 0.25) (layer F.Cu) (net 5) (status 30))
 (segment (start 30.35 26.5) (end 30.5 26.65) (width 0.25) (layer F.Cu) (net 5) (status 30))
 (segment (start 40.5 19.1) (end 40.5 22.15) (width 0.25) (layer F.Cu) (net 5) (status 30))
 (segment (start 40.5 22.15) (end 40.15 22.5) (width 0.25) (layer F.Cu) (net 5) (status 30))
 (segment (start 44.25 19.33) (end 47.08 19.33) (width 0.25) (layer F.Cu) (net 6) (status 30))
 (segment (start 47.08 19.33) (end 47.25 19.5) (width 0.25) (layer F.Cu) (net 6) (status 30))
 (segment (start 44.25 19.33) (end 43.43 19.33) (width 0.25) (layer F.Cu) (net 6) (status 30))
 (segment (start 43.43 19.33) (end 40.5 16.4) (width 0.25) (layer F.Cu) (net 6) (status 30))
 (segment (start 40.5 16.4) (end 40.35 16.4) (width 0.25) (layer F.Cu) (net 6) (status 30))
 (segment (start 40.35 16.4) (end 38 18.75) (width 0.25) (layer F.Cu) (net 6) (status 10))
 (segment (start 38 18.75) (end 37 18.75) (width 0.25) (layer F.Cu) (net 6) (status 20))
 (segment (start 36.6 14.5) (end 38.25 14.5) (width 0.25) (layer F.Cu) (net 8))
 (segment (start 38.5 14.25) (end 44.25 14.25) (width 0.25) (layer F.Cu) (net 8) (status 30))
 (segment (start 38.25 14.5) (end 38.5 14.25) (width 0.25) (layer F.Cu) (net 8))
 (segment (start 37.1 16.5) (end 38.75 16.5) (width 0.25) (layer F.Cu) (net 9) (status 10))
 (segment (start 39.04 16.79) (end 44.25 16.79) (width 0.25) (layer B.Cu) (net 9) (status 20))
 (segment (start 38.75 16.5) (end 39.04 16.79) (width 0.25) (layer B.Cu) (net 9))
 (via (at 38.75 16.5) (size 0.6) (drill 0.4) (layers F.Cu B.Cu) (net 9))
 (segment (start 15.8 26.345) (end 15.8 23.55) (width 0.25) (layer F.Cu) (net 10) (status 30))
 (segment (start 15.8 23.55) (end 16.35 23) (width 0.25) (layer F.Cu) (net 10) (status 30))
 (segment (start 21.2 26.345) (end 21.2 24.55) (width 0.25) (layer F.Cu) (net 11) (status 10))
 (segment (start 28.5 27.5) (end 28.5 29.35) (width 0.25) (layer F.Cu) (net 11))
 (via (at 28.5 27.5) (size 0.6) (drill 0.4) (layers F.Cu B.Cu) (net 11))
 (segment (start 28.5 24.5) (end 28.5 27.5) (width 0.25) (layer B.Cu) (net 11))
 (segment (start 27.75 23.75) (end 28.5 24.5) (width 0.25) (layer B.Cu) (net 11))
 (segment (start 22 23.75) (end 27.75 23.75) (width 0.25) (layer B.Cu) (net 11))
 (via (at 22 23.75) (size 0.6) (drill 0.4) (layers F.Cu B.Cu) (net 11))
 (segment (start 21.2 24.55) (end 22 23.75) (width 0.25) (layer F.Cu) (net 11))
 (segment (start 30.5 29.35) (end 28.5 29.35) (width 0.25) (layer F.Cu) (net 11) (status 10))
 (segment (start 28.5 29.35) (end 26.45 29.35) (width 0.25) (layer F.Cu) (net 11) (status 20))
 (segment (start 26.45 29.35) (end 26.35 29.25) (width 0.25) (layer F.Cu) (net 11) (status 30))
 (segment (start 15.425 18.55) (end 16.95 18.55) (width 0.25) (layer B.Cu) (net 7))
 (segment (start 17.5 19) (end 20.03 19) (width 0.25) (layer F.Cu) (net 7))
 (segment (start 17 18.5) (end 17.5 19) (width 0.25) (layer F.Cu) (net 7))
 (via (at 17 18.5) (size 0.6) (drill 0.4) (layers F.Cu B.Cu) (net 7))
 (segment (start 16.95 18.55) (end 17 18.5) (width 0.25) (layer B.Cu) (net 7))
 (segment (start 13.65 23) (end 14 23) (width 0.25) (layer F.Cu) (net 7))
 (segment (start 14 23) (end 18 19) (width 0.25) (layer F.Cu) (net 7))
 (segment (start 18 19) (end 20.03 19) (width 0.25) (layer F.Cu) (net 7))
 (segment (start 15.8 27.615) (end 14.865 27.615) (width 0.25) (layer F.Cu) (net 7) (status 10))
 (segment (start 13.65 26.4) (end 13.65 23) (width 0.25) (layer F.Cu) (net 7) (status 20))
 (segment (start 14.865 27.615) (end 13.65 26.4) (width 0.25) (layer F.Cu) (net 7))
 (segment (start 20.03 19) (end 18.71 19) (width 0.25) (layer F.Cu) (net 7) (status 30)))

